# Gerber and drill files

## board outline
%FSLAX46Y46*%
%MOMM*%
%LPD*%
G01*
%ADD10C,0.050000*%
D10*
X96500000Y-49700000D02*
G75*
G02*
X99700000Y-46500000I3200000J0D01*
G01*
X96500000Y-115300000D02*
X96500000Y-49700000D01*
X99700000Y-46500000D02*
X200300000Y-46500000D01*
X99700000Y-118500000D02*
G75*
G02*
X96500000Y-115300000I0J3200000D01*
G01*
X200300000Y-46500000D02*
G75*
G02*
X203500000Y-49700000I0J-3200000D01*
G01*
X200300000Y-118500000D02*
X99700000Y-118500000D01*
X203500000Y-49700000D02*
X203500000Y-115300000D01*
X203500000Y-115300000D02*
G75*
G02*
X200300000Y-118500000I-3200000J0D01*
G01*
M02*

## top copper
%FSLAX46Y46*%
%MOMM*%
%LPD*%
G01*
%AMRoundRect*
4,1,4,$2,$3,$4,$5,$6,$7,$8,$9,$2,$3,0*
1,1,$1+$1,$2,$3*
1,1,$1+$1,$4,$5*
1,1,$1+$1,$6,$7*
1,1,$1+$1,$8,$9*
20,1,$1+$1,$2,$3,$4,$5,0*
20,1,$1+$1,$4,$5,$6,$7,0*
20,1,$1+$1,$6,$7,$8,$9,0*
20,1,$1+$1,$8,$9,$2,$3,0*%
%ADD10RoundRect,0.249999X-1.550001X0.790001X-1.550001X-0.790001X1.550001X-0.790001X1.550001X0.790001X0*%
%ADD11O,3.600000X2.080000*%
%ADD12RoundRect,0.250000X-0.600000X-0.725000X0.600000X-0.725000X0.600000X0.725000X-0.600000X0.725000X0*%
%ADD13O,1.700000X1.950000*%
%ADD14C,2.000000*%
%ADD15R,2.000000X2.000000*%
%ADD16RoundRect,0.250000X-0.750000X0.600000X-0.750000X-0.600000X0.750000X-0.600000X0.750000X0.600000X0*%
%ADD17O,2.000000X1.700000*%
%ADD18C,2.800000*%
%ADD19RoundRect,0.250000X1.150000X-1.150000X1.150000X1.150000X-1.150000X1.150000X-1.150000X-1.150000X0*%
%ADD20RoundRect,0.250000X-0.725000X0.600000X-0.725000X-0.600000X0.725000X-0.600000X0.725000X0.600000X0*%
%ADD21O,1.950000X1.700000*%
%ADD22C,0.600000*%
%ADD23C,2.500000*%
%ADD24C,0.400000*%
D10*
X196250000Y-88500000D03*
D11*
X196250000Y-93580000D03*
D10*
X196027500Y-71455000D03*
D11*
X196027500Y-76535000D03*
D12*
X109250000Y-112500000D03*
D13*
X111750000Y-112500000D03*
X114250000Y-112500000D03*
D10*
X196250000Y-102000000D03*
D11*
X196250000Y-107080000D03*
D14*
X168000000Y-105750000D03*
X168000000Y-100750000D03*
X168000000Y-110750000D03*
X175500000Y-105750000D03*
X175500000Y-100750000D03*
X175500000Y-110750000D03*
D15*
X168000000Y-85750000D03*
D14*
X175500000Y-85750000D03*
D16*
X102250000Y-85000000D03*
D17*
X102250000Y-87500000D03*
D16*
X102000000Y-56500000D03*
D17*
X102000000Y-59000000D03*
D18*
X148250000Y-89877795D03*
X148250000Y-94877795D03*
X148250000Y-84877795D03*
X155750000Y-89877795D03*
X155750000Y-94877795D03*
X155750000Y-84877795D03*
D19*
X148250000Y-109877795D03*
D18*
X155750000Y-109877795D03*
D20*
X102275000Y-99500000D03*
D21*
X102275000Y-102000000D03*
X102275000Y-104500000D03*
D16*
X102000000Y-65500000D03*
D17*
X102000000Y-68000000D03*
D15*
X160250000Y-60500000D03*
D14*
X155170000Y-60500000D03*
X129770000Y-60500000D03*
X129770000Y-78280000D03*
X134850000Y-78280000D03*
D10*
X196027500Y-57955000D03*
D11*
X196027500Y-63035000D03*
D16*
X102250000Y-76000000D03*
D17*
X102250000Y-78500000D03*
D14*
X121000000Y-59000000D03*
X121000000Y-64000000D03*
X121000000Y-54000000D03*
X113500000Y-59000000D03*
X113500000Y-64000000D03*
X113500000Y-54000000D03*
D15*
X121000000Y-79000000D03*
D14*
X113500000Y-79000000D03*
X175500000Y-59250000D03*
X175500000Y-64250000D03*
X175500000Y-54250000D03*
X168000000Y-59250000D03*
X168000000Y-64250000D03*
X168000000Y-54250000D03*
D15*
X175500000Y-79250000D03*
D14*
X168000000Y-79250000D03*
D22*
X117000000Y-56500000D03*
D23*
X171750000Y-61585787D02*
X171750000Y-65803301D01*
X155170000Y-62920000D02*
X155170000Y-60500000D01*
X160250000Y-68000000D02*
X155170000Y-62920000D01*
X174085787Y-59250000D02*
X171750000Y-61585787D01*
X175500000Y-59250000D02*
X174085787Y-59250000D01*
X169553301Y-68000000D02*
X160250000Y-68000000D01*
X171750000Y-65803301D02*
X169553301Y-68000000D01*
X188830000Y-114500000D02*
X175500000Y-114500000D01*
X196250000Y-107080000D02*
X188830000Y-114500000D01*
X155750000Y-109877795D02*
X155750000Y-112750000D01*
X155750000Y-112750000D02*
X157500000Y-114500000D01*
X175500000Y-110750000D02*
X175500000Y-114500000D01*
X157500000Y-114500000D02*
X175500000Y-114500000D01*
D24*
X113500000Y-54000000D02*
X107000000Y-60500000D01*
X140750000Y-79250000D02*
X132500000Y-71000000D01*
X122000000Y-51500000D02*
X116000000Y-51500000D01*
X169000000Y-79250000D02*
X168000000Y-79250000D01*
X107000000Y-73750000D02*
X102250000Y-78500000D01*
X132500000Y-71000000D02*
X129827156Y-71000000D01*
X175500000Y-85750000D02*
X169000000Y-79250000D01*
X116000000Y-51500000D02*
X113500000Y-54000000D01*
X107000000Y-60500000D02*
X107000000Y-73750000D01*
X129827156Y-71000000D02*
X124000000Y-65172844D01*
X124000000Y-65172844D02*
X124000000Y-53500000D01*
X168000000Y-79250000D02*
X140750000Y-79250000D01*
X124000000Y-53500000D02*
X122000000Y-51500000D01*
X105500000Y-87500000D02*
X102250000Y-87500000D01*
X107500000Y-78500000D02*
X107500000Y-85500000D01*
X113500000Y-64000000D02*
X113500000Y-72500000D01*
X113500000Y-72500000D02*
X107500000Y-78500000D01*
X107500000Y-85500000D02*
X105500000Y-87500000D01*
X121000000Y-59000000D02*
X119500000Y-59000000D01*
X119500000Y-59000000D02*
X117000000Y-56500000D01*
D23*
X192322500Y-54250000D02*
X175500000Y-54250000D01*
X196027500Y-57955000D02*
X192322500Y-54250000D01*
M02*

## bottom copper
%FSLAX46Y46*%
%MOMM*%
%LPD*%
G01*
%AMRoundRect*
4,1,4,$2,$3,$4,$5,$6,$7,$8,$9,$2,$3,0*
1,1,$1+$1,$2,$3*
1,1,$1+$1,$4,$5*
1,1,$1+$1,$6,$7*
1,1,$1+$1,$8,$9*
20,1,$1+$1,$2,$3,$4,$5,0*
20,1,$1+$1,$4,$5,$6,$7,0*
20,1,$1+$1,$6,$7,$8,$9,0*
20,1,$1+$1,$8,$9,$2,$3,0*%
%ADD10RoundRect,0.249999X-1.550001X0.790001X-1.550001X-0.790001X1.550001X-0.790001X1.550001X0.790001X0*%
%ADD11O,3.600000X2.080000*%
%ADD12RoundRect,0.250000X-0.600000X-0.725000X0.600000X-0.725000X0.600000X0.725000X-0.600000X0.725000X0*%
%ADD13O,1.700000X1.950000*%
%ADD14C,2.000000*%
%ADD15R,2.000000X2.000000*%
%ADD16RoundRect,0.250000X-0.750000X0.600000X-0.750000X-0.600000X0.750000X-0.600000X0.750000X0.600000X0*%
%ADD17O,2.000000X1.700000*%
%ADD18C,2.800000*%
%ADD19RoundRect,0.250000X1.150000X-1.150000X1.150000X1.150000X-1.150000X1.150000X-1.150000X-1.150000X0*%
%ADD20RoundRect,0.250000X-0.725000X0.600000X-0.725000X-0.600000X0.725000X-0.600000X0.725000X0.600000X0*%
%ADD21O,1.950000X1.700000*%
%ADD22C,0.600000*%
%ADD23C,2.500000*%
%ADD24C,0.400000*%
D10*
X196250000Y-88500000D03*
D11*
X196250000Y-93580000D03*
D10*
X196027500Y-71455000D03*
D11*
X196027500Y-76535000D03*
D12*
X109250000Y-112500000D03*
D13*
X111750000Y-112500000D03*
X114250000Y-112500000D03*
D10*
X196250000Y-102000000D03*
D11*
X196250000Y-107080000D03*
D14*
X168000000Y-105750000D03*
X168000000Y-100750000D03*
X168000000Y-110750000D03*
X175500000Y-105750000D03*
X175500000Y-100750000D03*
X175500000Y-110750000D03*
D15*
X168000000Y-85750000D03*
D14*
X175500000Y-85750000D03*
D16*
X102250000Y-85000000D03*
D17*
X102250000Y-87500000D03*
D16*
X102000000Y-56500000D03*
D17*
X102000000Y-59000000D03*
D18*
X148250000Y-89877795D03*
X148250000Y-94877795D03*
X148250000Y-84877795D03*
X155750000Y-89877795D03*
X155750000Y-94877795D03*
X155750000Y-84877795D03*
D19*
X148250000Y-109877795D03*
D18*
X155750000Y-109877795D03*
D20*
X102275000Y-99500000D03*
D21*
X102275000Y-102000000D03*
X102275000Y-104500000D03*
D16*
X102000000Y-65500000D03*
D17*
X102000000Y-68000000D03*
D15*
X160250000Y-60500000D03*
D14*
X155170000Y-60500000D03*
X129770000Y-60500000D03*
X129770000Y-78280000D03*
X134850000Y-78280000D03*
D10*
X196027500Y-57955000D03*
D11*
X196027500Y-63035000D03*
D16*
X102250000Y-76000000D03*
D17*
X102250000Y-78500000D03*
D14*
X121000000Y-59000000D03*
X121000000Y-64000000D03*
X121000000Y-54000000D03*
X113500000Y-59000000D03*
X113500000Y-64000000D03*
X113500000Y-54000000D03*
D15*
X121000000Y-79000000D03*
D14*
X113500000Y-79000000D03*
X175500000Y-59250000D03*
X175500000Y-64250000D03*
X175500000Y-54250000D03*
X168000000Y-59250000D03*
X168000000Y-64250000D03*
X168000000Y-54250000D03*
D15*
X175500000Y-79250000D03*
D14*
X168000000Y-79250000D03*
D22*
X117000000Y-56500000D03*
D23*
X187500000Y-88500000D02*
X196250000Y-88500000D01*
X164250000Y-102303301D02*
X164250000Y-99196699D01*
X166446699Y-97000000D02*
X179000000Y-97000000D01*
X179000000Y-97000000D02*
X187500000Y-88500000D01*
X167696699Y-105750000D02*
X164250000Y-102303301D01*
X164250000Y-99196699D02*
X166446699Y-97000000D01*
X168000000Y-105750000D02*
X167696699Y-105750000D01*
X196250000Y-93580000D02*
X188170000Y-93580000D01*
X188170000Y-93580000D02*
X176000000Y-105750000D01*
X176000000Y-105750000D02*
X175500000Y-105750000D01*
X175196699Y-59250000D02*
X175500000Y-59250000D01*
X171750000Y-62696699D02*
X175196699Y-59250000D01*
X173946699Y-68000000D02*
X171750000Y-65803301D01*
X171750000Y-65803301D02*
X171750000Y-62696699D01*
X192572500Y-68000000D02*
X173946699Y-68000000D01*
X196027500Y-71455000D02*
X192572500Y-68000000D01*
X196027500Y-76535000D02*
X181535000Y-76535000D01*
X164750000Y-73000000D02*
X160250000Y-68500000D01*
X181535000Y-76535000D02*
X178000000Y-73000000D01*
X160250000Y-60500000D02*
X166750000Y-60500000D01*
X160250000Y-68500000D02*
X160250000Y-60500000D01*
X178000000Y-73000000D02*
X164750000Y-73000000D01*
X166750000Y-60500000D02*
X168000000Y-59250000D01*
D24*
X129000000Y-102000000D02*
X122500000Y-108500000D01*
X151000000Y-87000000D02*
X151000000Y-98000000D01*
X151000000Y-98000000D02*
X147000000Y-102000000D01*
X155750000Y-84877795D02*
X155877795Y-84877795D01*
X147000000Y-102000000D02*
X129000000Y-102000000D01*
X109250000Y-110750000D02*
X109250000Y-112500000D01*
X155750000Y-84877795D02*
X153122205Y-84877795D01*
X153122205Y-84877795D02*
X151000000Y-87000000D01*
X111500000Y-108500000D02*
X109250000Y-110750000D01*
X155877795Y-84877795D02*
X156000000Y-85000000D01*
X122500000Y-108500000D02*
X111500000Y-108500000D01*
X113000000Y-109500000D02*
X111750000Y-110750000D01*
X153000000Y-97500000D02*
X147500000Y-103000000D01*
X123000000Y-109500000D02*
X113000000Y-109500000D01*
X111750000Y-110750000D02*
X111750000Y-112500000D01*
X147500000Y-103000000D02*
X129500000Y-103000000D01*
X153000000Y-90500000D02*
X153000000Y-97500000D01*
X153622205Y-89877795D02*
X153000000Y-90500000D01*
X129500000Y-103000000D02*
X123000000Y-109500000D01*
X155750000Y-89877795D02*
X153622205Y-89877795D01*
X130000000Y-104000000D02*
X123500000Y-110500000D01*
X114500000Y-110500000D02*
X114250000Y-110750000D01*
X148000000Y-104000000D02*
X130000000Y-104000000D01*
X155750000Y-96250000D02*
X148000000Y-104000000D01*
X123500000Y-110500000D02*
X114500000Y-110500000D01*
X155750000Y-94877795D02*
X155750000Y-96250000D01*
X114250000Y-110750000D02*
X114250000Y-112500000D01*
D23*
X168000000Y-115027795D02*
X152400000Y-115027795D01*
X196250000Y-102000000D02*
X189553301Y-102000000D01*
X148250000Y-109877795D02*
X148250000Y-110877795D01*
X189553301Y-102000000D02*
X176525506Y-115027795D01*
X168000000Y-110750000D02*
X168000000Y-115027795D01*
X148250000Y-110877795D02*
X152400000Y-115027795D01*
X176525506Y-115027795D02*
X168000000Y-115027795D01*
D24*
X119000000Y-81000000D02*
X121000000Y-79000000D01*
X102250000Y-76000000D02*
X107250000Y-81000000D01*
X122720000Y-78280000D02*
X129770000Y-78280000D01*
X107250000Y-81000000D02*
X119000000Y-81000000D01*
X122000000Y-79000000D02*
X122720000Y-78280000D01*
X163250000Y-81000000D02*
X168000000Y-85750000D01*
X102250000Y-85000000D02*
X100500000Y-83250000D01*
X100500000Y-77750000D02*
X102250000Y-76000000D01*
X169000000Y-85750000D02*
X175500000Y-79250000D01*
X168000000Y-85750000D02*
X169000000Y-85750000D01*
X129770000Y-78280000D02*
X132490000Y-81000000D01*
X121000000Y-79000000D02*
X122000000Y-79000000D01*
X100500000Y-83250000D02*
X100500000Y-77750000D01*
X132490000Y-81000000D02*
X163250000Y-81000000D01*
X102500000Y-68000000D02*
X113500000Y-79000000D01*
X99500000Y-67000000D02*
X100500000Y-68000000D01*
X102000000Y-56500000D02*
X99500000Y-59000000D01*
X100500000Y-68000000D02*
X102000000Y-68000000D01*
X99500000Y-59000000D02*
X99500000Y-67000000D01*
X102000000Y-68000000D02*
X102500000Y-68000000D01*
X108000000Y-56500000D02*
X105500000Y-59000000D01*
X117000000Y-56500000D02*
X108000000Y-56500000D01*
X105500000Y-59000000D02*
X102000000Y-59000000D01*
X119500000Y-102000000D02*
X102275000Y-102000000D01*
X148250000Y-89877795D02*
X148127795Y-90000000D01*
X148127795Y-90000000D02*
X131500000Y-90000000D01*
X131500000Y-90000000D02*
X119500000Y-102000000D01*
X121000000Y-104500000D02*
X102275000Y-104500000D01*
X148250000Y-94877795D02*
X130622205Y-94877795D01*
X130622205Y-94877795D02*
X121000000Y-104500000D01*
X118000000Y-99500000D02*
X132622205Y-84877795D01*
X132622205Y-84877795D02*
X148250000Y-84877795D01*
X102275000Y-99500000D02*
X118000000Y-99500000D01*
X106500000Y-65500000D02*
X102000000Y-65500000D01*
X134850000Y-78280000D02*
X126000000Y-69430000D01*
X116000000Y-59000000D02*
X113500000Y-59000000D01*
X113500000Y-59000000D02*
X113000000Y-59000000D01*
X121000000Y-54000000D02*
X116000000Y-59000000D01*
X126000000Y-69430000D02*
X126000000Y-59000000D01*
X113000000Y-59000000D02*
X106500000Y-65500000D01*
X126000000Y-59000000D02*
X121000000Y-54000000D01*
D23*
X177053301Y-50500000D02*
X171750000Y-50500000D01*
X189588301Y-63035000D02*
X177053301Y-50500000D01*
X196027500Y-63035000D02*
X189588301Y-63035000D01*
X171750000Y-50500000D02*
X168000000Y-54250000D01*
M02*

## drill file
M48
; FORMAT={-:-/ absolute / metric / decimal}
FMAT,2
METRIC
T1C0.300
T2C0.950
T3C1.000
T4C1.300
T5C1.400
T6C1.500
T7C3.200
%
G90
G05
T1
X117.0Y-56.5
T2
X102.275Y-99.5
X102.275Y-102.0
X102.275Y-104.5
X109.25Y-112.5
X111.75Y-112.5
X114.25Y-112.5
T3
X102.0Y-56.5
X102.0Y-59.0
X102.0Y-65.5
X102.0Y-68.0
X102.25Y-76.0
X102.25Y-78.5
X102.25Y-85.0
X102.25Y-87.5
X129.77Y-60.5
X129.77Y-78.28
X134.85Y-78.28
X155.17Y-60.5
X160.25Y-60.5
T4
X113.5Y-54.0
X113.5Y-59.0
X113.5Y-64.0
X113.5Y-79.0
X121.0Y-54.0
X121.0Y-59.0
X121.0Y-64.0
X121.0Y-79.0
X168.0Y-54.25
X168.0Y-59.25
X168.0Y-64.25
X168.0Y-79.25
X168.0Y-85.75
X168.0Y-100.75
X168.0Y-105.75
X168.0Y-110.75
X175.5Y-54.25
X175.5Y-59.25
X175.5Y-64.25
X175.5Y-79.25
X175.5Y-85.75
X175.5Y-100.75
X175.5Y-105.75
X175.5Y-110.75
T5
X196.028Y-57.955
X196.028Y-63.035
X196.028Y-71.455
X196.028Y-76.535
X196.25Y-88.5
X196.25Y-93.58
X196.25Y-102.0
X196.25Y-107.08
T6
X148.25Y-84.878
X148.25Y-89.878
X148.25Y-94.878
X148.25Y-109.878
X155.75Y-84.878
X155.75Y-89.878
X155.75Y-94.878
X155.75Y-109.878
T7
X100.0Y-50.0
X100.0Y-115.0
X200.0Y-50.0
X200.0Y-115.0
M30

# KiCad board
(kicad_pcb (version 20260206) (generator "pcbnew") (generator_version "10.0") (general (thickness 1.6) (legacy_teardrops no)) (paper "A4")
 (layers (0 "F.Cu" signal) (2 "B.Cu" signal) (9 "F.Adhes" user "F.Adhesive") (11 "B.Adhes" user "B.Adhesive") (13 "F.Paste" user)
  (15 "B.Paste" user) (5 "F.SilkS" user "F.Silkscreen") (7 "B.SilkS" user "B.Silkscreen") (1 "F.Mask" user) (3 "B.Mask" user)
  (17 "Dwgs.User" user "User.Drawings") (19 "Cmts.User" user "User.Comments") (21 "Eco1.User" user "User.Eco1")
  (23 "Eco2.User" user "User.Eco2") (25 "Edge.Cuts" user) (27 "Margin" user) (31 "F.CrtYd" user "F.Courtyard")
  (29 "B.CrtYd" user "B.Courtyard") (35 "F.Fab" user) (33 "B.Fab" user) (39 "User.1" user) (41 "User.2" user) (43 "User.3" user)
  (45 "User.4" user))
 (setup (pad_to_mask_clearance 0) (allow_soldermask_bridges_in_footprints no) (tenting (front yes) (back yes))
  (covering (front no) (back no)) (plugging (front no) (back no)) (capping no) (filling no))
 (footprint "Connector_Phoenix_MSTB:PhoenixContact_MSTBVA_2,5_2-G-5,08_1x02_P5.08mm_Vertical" (layer "F.Cu") (at 196.25 88.5 -90)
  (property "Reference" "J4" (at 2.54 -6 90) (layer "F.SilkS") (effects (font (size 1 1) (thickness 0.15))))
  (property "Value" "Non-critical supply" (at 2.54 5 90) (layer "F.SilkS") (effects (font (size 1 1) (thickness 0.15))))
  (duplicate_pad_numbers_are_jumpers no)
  (pad "1" thru_hole roundrect (at 0 0 270) (size 2.08 3.6) (drill 1.4) (layers "*.Cu" "*.Mask") (remove_unused_layers no)
   (roundrect_rratio 0.120192) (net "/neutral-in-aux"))
  (pad "2" thru_hole oval (at 5.08 0 270) (size 2.08 3.6) (drill 1.4) (layers "*.Cu" "*.Mask") (remove_unused_layers no)
   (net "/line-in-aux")))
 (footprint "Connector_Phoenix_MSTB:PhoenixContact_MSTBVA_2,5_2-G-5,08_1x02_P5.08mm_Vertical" (layer "F.Cu") (at 196.0275 71.455 -90)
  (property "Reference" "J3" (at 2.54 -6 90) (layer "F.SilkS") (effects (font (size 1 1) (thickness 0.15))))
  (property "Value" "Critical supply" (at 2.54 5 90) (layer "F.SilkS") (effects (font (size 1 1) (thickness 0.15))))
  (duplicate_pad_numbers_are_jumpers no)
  (pad "1" thru_hole roundrect (at 0 0 270) (size 2.08 3.6) (drill 1.4) (layers "*.Cu" "*.Mask") (remove_unused_layers no)
   (roundrect_rratio 0.120192) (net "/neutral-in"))
  (pad "2" thru_hole oval (at 5.08 0 270) (size 2.08 3.6) (drill 1.4) (layers "*.Cu" "*.Mask") (remove_unused_layers no) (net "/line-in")))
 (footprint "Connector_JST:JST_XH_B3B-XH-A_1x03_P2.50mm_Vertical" (layer "F.Cu") (at 109.25 112.5)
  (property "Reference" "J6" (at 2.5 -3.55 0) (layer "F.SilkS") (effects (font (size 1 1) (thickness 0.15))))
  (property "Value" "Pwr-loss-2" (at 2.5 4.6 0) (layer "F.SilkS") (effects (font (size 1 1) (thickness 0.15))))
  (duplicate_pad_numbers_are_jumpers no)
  (pad "1" thru_hole roundrect (at 0 0) (size 1.7 1.95) (drill 0.95) (layers "*.Cu" "*.Mask") (remove_unused_layers no)
   (roundrect_rratio 0.147059) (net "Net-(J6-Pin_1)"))
  (pad "2" thru_hole oval (at 2.5 0) (size 1.7 1.95) (drill 0.95) (layers "*.Cu" "*.Mask") (remove_unused_layers no) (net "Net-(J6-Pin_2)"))
  (pad "3" thru_hole oval (at 5 0) (size 1.7 1.95) (drill 0.95) (layers "*.Cu" "*.Mask") (remove_unused_layers no) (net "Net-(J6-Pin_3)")))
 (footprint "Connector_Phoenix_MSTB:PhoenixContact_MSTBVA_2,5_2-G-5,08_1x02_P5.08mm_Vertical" (layer "F.Cu") (at 196.25 102 -90)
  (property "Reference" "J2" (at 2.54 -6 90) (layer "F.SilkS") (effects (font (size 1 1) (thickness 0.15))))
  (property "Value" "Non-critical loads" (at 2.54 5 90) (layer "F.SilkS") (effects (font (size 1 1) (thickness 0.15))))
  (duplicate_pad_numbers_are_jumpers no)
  (pad "1" thru_hole roundrect (at 0 0 270) (size 2.08 3.6) (drill 1.4) (layers "*.Cu" "*.Mask") (remove_unused_layers no)
   (roundrect_rratio 0.120192) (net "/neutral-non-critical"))
  (pad "2" thru_hole oval (at 5.08 0 270) (size 2.08 3.6) (drill 1.4) (layers "*.Cu" "*.Mask") (remove_unused_layers no)
   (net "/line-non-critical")))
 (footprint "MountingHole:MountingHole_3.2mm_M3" (layer "F.Cu") (at 200 50)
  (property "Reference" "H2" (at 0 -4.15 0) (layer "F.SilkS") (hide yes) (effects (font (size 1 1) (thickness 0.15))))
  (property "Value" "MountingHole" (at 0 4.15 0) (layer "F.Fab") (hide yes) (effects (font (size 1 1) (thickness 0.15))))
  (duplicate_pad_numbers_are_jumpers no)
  (pad "" np_thru_hole circle (at 0 0) (size 3.2 3.2) (drill 3.2) (layers "*.Cu" "*.Mask")))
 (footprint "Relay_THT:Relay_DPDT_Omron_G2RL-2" (layer "F.Cu") (at 168 85.75)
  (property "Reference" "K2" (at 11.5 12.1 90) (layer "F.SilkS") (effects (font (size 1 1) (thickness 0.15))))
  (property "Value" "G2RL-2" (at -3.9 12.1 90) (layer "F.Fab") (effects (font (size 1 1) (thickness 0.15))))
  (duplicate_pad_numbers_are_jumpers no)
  (pad "11" thru_hole circle (at 0 20) (size 2 2) (drill 1.3) (layers "*.Cu" "*.Mask") (remove_unused_layers no) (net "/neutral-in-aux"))
  (pad "12" thru_hole circle (at 0 15) (size 2 2) (drill 1.3) (layers "*.Cu" "*.Mask") (remove_unused_layers no)
   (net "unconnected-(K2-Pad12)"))
  (pad "14" thru_hole circle (at 0 25) (size 2 2) (drill 1.3) (layers "*.Cu" "*.Mask") (remove_unused_layers no)
   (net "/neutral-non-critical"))
  (pad "21" thru_hole circle (at 7.5 20) (size 2 2) (drill 1.3) (layers "*.Cu" "*.Mask") (remove_unused_layers no) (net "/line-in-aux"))
  (pad "22" thru_hole circle (at 7.5 15) (size 2 2) (drill 1.3) (layers "*.Cu" "*.Mask") (remove_unused_layers no)
   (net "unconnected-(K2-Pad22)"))
  (pad "24" thru_hole circle (at 7.5 25) (size 2 2) (drill 1.3) (layers "*.Cu" "*.Mask") (remove_unused_layers no)
   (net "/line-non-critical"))
  (pad "A1" thru_hole rect (at 0 0) (size 2 2) (drill 1.3) (layers "*.Cu" "*.Mask") (remove_unused_layers no) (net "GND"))
  (pad "A2" thru_hole circle (at 7.5 0) (size 2 2) (drill 1.3) (layers "*.Cu" "*.Mask") (remove_unused_layers no) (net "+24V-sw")))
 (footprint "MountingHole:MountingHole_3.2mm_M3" (layer "F.Cu") (at 100 50)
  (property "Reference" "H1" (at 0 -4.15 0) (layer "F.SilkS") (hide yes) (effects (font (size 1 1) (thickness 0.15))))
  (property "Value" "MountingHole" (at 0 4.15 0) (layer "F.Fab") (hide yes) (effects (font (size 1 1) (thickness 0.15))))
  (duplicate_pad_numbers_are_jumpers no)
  (pad "" np_thru_hole circle (at 0 0) (size 3.2 3.2) (drill 3.2) (layers "*.Cu" "*.Mask")))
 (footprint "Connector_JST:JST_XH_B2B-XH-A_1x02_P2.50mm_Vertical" (layer "F.Cu") (at 102.25 85 -90)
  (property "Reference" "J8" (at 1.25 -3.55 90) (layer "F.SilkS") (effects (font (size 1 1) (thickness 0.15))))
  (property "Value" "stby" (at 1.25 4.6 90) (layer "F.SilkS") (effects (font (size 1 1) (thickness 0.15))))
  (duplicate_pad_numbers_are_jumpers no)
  (pad "1" thru_hole roundrect (at 0 0 270) (size 1.7 2) (drill 1) (layers "*.Cu" "*.Mask") (remove_unused_layers no)
   (roundrect_rratio 0.147059) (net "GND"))
  (pad "2" thru_hole oval (at 2.5 0 270) (size 1.7 2) (drill 1) (layers "*.Cu" "*.Mask") (remove_unused_layers no) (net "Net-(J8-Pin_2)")))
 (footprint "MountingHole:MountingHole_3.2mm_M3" (layer "F.Cu") (at 200 115)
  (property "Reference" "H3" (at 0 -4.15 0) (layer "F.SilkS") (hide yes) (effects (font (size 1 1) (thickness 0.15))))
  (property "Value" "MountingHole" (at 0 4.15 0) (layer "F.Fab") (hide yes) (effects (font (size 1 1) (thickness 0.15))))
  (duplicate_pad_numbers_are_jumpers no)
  (pad "" np_thru_hole circle (at 0 0) (size 3.2 3.2) (drill 3.2) (layers "*.Cu" "*.Mask")))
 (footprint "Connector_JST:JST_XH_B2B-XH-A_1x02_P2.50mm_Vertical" (layer "F.Cu") (at 102 56.5 -90)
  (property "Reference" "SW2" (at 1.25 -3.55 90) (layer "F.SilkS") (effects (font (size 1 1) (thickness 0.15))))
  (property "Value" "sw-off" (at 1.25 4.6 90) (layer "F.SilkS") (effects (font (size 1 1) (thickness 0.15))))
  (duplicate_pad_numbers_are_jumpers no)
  (pad "1" thru_hole roundrect (at 0 0 270) (size 1.7 2) (drill 1) (layers "*.Cu" "*.Mask") (remove_unused_layers no)
   (roundrect_rratio 0.147059) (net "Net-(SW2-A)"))
  (pad "2" thru_hole oval (at 2.5 0 270) (size 1.7 2) (drill 1) (layers "*.Cu" "*.Mask") (remove_unused_layers no) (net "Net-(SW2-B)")))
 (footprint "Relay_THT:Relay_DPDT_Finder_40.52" (layer "F.Cu") (at 148.25 109.877795 90)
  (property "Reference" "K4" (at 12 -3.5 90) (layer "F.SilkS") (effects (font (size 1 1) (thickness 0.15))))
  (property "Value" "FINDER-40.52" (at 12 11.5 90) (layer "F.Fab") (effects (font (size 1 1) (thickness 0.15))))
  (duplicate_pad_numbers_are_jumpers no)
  (pad "11" thru_hole circle (at 20 0 90) (size 2.8 2.8) (drill 1.5) (layers "*.Cu" "*.Mask") (remove_unused_layers no)
   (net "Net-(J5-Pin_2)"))
  (pad "12" thru_hole circle (at 15 0 90) (size 2.8 2.8) (drill 1.5) (layers "*.Cu" "*.Mask") (remove_unused_layers no)
   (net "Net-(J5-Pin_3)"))
  (pad "14" thru_hole circle (at 25 0 90) (size 2.8 2.8) (drill 1.5) (layers "*.Cu" "*.Mask") (remove_unused_layers no)
   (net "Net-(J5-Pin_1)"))
  (pad "21" thru_hole circle (at 20 7.5 90) (size 2.8 2.8) (drill 1.5) (layers "*.Cu" "*.Mask") (remove_unused_layers no)
   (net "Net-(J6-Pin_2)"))
  (pad "22" thru_hole circle (at 15 7.5 90) (size 2.8 2.8) (drill 1.5) (layers "*.Cu" "*.Mask") (remove_unused_layers no)
   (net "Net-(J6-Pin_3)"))
  (pad "24" thru_hole circle (at 25 7.5 90) (size 2.8 2.8) (drill 1.5) (layers "*.Cu" "*.Mask") (remove_unused_layers no)
   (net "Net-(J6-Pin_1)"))
  (pad "A1" thru_hole roundrect (at 0 0 90) (size 2.8 2.8) (drill 1.5) (layers "*.Cu" "*.Mask") (remove_unused_layers no)
   (roundrect_rratio 0.08928571429) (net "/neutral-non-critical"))
  (pad "A2" thru_hole circle (at 0 7.5 90) (size 2.8 2.8) (drill 1.5) (layers "*.Cu" "*.Mask") (remove_unused_layers no)
   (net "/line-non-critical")))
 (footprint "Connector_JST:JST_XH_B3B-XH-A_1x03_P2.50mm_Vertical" (layer "F.Cu") (at 102.275 99.5 -90)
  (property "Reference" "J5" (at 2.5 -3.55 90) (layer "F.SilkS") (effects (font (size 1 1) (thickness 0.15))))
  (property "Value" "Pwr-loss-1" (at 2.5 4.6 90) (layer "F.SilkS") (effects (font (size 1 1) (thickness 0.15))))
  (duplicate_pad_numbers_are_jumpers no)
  (pad "1" thru_hole roundrect (at 0 0 270) (size 1.7 1.95) (drill 0.95) (layers "*.Cu" "*.Mask") (remove_unused_layers no)
   (roundrect_rratio 0.147059) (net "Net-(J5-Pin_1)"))
  (pad "2" thru_hole oval (at 2.5 0 270) (size 1.7 1.95) (drill 0.95) (layers "*.Cu" "*.Mask") (remove_unused_layers no)
   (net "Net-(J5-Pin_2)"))
  (pad "3" thru_hole oval (at 5 0 270) (size 1.7 1.95) (drill 0.95) (layers "*.Cu" "*.Mask") (remove_unused_layers no)
   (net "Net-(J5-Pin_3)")))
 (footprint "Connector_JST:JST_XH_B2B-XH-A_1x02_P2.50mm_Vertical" (layer "F.Cu") (at 102 65.5 -90)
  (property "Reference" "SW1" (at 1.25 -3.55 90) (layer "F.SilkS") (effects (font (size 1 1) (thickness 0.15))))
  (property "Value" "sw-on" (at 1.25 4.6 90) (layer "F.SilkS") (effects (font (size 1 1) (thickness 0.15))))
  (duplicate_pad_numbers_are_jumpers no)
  (pad "1" thru_hole roundrect (at 0 0 270) (size 1.7 2) (drill 1) (layers "*.Cu" "*.Mask") (remove_unused_layers no)
   (roundrect_rratio 0.147059) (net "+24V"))
  (pad "2" thru_hole oval (at 2.5 0 270) (size 1.7 2) (drill 1) (layers "*.Cu" "*.Mask") (remove_unused_layers no) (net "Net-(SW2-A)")))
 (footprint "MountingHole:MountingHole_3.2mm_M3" (layer "F.Cu") (at 100 115)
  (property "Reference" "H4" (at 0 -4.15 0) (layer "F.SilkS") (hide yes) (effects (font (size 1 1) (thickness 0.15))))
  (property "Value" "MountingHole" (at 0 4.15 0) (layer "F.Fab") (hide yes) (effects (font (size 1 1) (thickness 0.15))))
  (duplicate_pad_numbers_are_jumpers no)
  (pad "" np_thru_hole circle (at 0 0) (size 3.2 3.2) (drill 3.2) (layers "*.Cu" "*.Mask")))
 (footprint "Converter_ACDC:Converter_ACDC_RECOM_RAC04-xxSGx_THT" (layer "F.Cu") (at 160.25 60.5 -90)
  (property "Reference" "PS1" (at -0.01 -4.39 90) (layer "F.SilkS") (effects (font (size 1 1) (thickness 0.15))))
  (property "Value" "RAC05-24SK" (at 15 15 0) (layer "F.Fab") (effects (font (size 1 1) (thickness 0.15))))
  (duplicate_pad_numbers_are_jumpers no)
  (pad "1" thru_hole rect (at 0 0) (size 2 2) (drill 1) (layers "*.Cu" "*.Mask") (remove_unused_layers no) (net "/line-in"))
  (pad "2" thru_hole circle (at 0 5.08) (size 2 2) (drill 1) (layers "*.Cu" "*.Mask") (remove_unused_layers no) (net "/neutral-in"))
  (pad "3" thru_hole circle (at 0 30.48 90) (size 2 2) (drill 1) (layers "*.Cu" "*.Mask") (remove_unused_layers no)
   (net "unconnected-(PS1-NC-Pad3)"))
  (pad "4" thru_hole circle (at 17.78 30.48) (size 2 2) (drill 1) (layers "*.Cu" "*.Mask") (remove_unused_layers no) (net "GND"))
  (pad "5" thru_hole circle (at 17.78 25.4) (size 2 2) (drill 1) (layers "*.Cu" "*.Mask") (remove_unused_layers no) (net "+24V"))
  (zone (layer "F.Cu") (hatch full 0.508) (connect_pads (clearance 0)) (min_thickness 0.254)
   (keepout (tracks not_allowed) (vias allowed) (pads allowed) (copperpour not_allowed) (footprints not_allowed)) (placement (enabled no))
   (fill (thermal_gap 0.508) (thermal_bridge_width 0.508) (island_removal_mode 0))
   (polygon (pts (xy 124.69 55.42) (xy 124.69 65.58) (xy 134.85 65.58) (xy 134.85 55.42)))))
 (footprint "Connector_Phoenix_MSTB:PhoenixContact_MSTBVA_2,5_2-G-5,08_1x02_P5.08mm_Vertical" (layer "F.Cu") (at 196.0275 57.955 -90)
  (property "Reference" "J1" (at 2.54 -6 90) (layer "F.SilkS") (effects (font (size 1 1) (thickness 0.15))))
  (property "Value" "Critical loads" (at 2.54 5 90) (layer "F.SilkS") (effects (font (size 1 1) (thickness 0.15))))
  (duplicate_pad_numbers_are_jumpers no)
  (pad "1" thru_hole roundrect (at 0 0 270) (size 2.08 3.6) (drill 1.4) (layers "*.Cu" "*.Mask") (remove_unused_layers no)
   (roundrect_rratio 0.120192) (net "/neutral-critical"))
  (pad "2" thru_hole oval (at 5.08 0 270) (size 2.08 3.6) (drill 1.4) (layers "*.Cu" "*.Mask") (remove_unused_layers no)
   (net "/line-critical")))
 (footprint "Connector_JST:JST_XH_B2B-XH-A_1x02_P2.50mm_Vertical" (layer "F.Cu") (at 102.25 76 -90)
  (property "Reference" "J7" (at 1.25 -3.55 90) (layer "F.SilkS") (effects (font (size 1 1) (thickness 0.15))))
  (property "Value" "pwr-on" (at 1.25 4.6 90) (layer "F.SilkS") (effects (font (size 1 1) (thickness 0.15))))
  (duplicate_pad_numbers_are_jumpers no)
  (pad "1" thru_hole roundrect (at 0 0 270) (size 1.7 2) (drill 1) (layers "*.Cu" "*.Mask") (remove_unused_layers no)
   (roundrect_rratio 0.147059) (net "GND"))
  (pad "2" thru_hole oval (at 2.5 0 270) (size 1.7 2) (drill 1) (layers "*.Cu" "*.Mask") (remove_unused_layers no) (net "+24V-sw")))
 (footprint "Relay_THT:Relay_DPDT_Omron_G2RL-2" (layer "F.Cu") (at 121 79 180)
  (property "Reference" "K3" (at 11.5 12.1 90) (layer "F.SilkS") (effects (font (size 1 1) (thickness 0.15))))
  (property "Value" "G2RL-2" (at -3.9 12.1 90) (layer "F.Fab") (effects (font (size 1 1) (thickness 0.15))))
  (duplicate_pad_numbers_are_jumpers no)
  (pad "11" thru_hole circle (at 0 20 180) (size 2 2) (drill 1.3) (layers "*.Cu" "*.Mask") (remove_unused_layers no) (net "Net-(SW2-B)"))
  (pad "12" thru_hole circle (at 0 15 180) (size 2 2) (drill 1.3) (layers "*.Cu" "*.Mask") (remove_unused_layers no)
   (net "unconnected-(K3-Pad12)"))
  (pad "14" thru_hole circle (at 0 25 180) (size 2 2) (drill 1.3) (layers "*.Cu" "*.Mask") (remove_unused_layers no) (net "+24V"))
  (pad "21" thru_hole circle (at 7.5 20 180) (size 2 2) (drill 1.3) (layers "*.Cu" "*.Mask") (remove_unused_layers no) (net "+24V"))
  (pad "22" thru_hole circle (at 7.5 15 180) (size 2 2) (drill 1.3) (layers "*.Cu" "*.Mask") (remove_unused_layers no)
   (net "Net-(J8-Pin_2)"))
  (pad "24" thru_hole circle (at 7.5 25 180) (size 2 2) (drill 1.3) (layers "*.Cu" "*.Mask") (remove_unused_layers no) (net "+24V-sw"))
  (pad "A1" thru_hole rect (at 0 0 180) (size 2 2) (drill 1.3) (layers "*.Cu" "*.Mask") (remove_unused_layers no) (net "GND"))
  (pad "A2" thru_hole circle (at 7.5 0 180) (size 2 2) (drill 1.3) (layers "*.Cu" "*.Mask") (remove_unused_layers no) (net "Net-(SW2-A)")))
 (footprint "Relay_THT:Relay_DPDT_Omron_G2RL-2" (layer "F.Cu") (at 175.5 79.25 180)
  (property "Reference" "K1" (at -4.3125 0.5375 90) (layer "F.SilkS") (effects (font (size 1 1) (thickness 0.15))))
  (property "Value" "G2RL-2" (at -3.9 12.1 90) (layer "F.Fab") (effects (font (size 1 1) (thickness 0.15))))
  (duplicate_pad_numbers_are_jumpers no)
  (pad "11" thru_hole circle (at 0 20 180) (size 2 2) (drill 1.3) (layers "*.Cu" "*.Mask") (remove_unused_layers no) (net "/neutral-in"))
  (pad "12" thru_hole circle (at 0 15 180) (size 2 2) (drill 1.3) (layers "*.Cu" "*.Mask") (remove_unused_layers no)
   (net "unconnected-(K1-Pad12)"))
  (pad "14" thru_hole circle (at 0 25 180) (size 2 2) (drill 1.3) (layers "*.Cu" "*.Mask") (remove_unused_layers no)
   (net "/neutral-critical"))
  (pad "21" thru_hole circle (at 7.5 20 180) (size 2 2) (drill 1.3) (layers "*.Cu" "*.Mask") (remove_unused_layers no) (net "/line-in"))
  (pad "22" thru_hole circle (at 7.5 15 180) (size 2 2) (drill 1.3) (layers "*.Cu" "*.Mask") (remove_unused_layers no)
   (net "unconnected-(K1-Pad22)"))
  (pad "24" thru_hole circle (at 7.5 25 180) (size 2 2) (drill 1.3) (layers "*.Cu" "*.Mask") (remove_unused_layers no)
   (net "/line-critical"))
  (pad "A1" thru_hole rect (at 0 0 180) (size 2 2) (drill 1.3) (layers "*.Cu" "*.Mask") (remove_unused_layers no) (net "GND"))
  (pad "A2" thru_hole circle (at 7.5 0 180) (size 2 2) (drill 1.3) (layers "*.Cu" "*.Mask") (remove_unused_layers no) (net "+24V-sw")))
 (gr_arc (start 96.5 49.7) (mid 97.437258 47.437258) (end 99.7 46.5) (stroke (width 0.05) (type default)) (layer "Edge.Cuts"))
 (gr_line (start 96.5 115.3) (end 96.5 49.7) (stroke (width 0.05) (type default)) (layer "Edge.Cuts"))
 (gr_line (start 99.7 46.5) (end 200.3 46.5) (stroke (width 0.05) (type default)) (layer "Edge.Cuts"))
 (gr_arc (start 99.7 118.5) (mid 97.437258 117.562742) (end 96.5 115.3) (stroke (width 0.05) (type default)) (layer "Edge.Cuts"))
 (gr_arc (start 200.3 46.5) (mid 202.562742 47.437258) (end 203.5 49.7) (stroke (width 0.05) (type default)) (layer "Edge.Cuts"))
 (gr_line (start 200.3 118.5) (end 99.7 118.5) (stroke (width 0.05) (type default)) (layer "Edge.Cuts"))
 (gr_line (start 203.5 49.7) (end 203.5 115.3) (stroke (width 0.05) (type default)) (layer "Edge.Cuts"))
 (gr_arc (start 203.5 115.3) (mid 202.562742 117.562742) (end 200.3 118.5) (stroke (width 0.05) (type default)) (layer "Edge.Cuts"))
 (segment (start 187.5 88.5) (end 196.25 88.5) (width 2.5) (layer "B.Cu") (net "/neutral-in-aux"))
 (segment (start 164.25 102.303301) (end 164.25 99.196699) (width 2.5) (layer "B.Cu") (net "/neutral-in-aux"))
 (segment (start 166.446699 97) (end 179 97) (width 2.5) (layer "B.Cu") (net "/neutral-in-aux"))
 (segment (start 179 97) (end 187.5 88.5) (width 2.5) (layer "B.Cu") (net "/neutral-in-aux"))
 (segment (start 167.696699 105.75) (end 164.25 102.303301) (width 2.5) (layer "B.Cu") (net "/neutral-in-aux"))
 (segment (start 164.25 99.196699) (end 166.446699 97) (width 2.5) (layer "B.Cu") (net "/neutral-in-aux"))
 (segment (start 168 105.75) (end 167.696699 105.75) (width 2.5) (layer "B.Cu") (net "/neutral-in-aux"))
 (segment (start 196.25 93.58) (end 188.17 93.58) (width 2.5) (layer "B.Cu") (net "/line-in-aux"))
 (segment (start 188.17 93.58) (end 176 105.75) (width 2.5) (layer "B.Cu") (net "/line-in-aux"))
 (segment (start 176 105.75) (end 175.5 105.75) (width 2.5) (layer "B.Cu") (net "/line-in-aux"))
 (segment (start 171.75 61.585787) (end 171.75 65.803301) (width 2.5) (layer "F.Cu") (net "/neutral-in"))
 (segment (start 155.17 62.92) (end 155.17 60.5) (width 2.5) (layer "F.Cu") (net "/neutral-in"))
 (segment (start 160.25 68) (end 155.17 62.92) (width 2.5) (layer "F.Cu") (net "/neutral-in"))
 (segment (start 174.085787 59.25) (end 171.75 61.585787) (width 2.5) (layer "F.Cu") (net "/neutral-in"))
 (segment (start 175.5 59.25) (end 174.085787 59.25) (width 2.5) (layer "F.Cu") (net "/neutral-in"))
 (segment (start 169.553301 68) (end 160.25 68) (width 2.5) (layer "F.Cu") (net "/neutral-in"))
 (segment (start 171.75 65.803301) (end 169.553301 68) (width 2.5) (layer "F.Cu") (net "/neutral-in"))
 (segment (start 175.196699 59.25) (end 175.5 59.25) (width 2.5) (layer "B.Cu") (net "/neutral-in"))
 (segment (start 171.75 62.696699) (end 175.196699 59.25) (width 2.5) (layer "B.Cu") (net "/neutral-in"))
 (segment (start 173.946699 68) (end 171.75 65.803301) (width 2.5) (layer "B.Cu") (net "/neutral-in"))
 (segment (start 171.75 65.803301) (end 171.75 62.696699) (width 2.5) (layer "B.Cu") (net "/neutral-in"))
 (segment (start 192.5725 68) (end 173.946699 68) (width 2.5) (layer "B.Cu") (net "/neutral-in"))
 (segment (start 196.0275 71.455) (end 192.5725 68) (width 2.5) (layer "B.Cu") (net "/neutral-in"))
 (segment (start 196.0275 76.535) (end 181.535 76.535) (width 2.5) (layer "B.Cu") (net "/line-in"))
 (segment (start 164.75 73) (end 160.25 68.5) (width 2.5) (layer "B.Cu") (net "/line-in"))
 (segment (start 181.535 76.535) (end 178 73) (width 2.5) (layer "B.Cu") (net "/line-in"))
 (segment (start 160.25 60.5) (end 166.75 60.5) (width 2.5) (layer "B.Cu") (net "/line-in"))
 (segment (start 160.25 68.5) (end 160.25 60.5) (width 2.5) (layer "B.Cu") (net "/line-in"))
 (segment (start 178 73) (end 164.75 73) (width 2.5) (layer "B.Cu") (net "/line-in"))
 (segment (start 166.75 60.5) (end 168 59.25) (width 2.5) (layer "B.Cu") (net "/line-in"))
 (segment (start 129 102) (end 122.5 108.5) (width 0.4) (layer "B.Cu") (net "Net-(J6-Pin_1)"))
 (segment (start 151 87) (end 151 98) (width 0.4) (layer "B.Cu") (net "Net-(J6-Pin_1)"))
 (segment (start 151 98) (end 147 102) (width 0.4) (layer "B.Cu") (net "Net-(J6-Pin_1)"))
 (segment (start 155.75 84.877795) (end 155.877795 84.877795) (width 0.4) (layer "B.Cu") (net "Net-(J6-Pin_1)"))
 (segment (start 147 102) (end 129 102) (width 0.4) (layer "B.Cu") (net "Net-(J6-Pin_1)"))
 (segment (start 109.25 110.75) (end 109.25 112.5) (width 0.4) (layer "B.Cu") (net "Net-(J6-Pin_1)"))
 (segment (start 155.75 84.877795) (end 153.122205 84.877795) (width 0.4) (layer "B.Cu") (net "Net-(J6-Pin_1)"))
 (segment (start 153.122205 84.877795) (end 151 87) (width 0.4) (layer "B.Cu") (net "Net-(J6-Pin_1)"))
 (segment (start 111.5 108.5) (end 109.25 110.75) (width 0.4) (layer "B.Cu") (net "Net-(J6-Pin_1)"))
 (segment (start 155.877795 84.877795) (end 156 85) (width 0.4) (layer "B.Cu") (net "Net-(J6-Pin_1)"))
 (segment (start 122.5 108.5) (end 111.5 108.5) (width 0.4) (layer "B.Cu") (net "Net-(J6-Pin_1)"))
 (segment (start 113 109.5) (end 111.75 110.75) (width 0.4) (layer "B.Cu") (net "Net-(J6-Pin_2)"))
 (segment (start 153 97.5) (end 147.5 103) (width 0.4) (layer "B.Cu") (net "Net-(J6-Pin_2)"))
 (segment (start 123 109.5) (end 113 109.5) (width 0.4) (layer "B.Cu") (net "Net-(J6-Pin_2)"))
 (segment (start 111.75 110.75) (end 111.75 112.5) (width 0.4) (layer "B.Cu") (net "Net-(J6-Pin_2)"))
 (segment (start 147.5 103) (end 129.5 103) (width 0.4) (layer "B.Cu") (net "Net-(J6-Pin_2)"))
 (segment (start 153 90.5) (end 153 97.5) (width 0.4) (layer "B.Cu") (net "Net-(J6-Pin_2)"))
 (segment (start 153.622205 89.877795) (end 153 90.5) (width 0.4) (layer "B.Cu") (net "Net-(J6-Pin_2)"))
 (segment (start 129.5 103) (end 123 109.5) (width 0.4) (layer "B.Cu") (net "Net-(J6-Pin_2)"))
 (segment (start 155.75 89.877795) (end 153.622205 89.877795) (width 0.4) (layer "B.Cu") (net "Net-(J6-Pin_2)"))
 (segment (start 130 104) (end 123.5 110.5) (width 0.4) (layer "B.Cu") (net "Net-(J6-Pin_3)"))
 (segment (start 114.5 110.5) (end 114.25 110.75) (width 0.4) (layer "B.Cu") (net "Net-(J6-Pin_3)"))
 (segment (start 148 104) (end 130 104) (width 0.4) (layer "B.Cu") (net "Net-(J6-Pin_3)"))
 (segment (start 155.75 96.25) (end 148 104) (width 0.4) (layer "B.Cu") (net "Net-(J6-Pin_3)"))
 (segment (start 123.5 110.5) (end 114.5 110.5) (width 0.4) (layer "B.Cu") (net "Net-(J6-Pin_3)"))
 (segment (start 155.75 94.877795) (end 155.75 96.25) (width 0.4) (layer "B.Cu") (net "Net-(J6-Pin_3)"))
 (segment (start 114.25 110.75) (end 114.25 112.5) (width 0.4) (layer "B.Cu") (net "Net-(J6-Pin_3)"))
 (segment (start 168 115.027795) (end 152.4 115.027795) (width 2.5) (layer "B.Cu") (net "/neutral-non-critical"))
 (segment (start 196.25 102) (end 189.553301 102) (width 2.5) (layer "B.Cu") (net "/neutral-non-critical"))
 (segment (start 148.25 109.877795) (end 148.25 110.877795) (width 2.5) (layer "B.Cu") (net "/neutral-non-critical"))
 (segment (start 189.553301 102) (end 176.525506 115.027795) (width 2.5) (layer "B.Cu") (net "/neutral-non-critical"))
 (segment (start 168 110.75) (end 168 115.027795) (width 2.5) (layer "B.Cu") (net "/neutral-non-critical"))
 (segment (start 148.25 110.877795) (end 152.4 115.027795) (width 2.5) (layer "B.Cu") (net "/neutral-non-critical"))
 (segment (start 176.525506 115.027795) (end 168 115.027795) (width 2.5) (layer "B.Cu") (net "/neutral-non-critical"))
 (segment (start 188.83 114.5) (end 175.5 114.5) (width 2.5) (layer "F.Cu") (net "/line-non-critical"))
 (segment (start 196.25 107.08) (end 188.83 114.5) (width 2.5) (layer "F.Cu") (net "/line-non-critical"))
 (segment (start 155.75 109.877795) (end 155.75 112.75) (width 2.5) (layer "F.Cu") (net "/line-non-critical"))
 (segment (start 155.75 112.75) (end 157.5 114.5) (width 2.5) (layer "F.Cu") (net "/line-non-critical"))
 (segment (start 175.5 110.75) (end 175.5 114.5) (width 2.5) (layer "F.Cu") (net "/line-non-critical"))
 (segment (start 157.5 114.5) (end 175.5 114.5) (width 2.5) (layer "F.Cu") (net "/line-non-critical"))
 (segment (start 119 81) (end 121 79) (width 0.4) (layer "B.Cu") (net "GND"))
 (segment (start 102.25 76) (end 107.25 81) (width 0.4) (layer "B.Cu") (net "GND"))
 (segment (start 122.72 78.28) (end 129.77 78.28) (width 0.4) (layer "B.Cu") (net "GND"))
 (segment (start 107.25 81) (end 119 81) (width 0.4) (layer "B.Cu") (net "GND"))
 (segment (start 122 79) (end 122.72 78.28) (width 0.4) (layer "B.Cu") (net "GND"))
 (segment (start 163.25 81) (end 168 85.75) (width 0.4) (layer "B.Cu") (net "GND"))
 (segment (start 102.25 85) (end 100.5 83.25) (width 0.4) (layer "B.Cu") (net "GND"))
 (segment (start 100.5 77.75) (end 102.25 76) (width 0.4) (layer "B.Cu") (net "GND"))
 (segment (start 169 85.75) (end 175.5 79.25) (width 0.4) (layer "B.Cu") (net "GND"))
 (segment (start 168 85.75) (end 169 85.75) (width 0.4) (layer "B.Cu") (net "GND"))
 (segment (start 129.77 78.28) (end 132.49 81) (width 0.4) (layer "B.Cu") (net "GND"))
 (segment (start 121 79) (end 122 79) (width 0.4) (layer "B.Cu") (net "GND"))
 (segment (start 100.5 83.25) (end 100.5 77.75) (width 0.4) (layer "B.Cu") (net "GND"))
 (segment (start 132.49 81) (end 163.25 81) (width 0.4) (layer "B.Cu") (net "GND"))
 (segment (start 113.5 54) (end 107 60.5) (width 0.4) (layer "F.Cu") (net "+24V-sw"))
 (segment (start 140.75 79.25) (end 132.5 71) (width 0.4) (layer "F.Cu") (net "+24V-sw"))
 (segment (start 122 51.5) (end 116 51.5) (width 0.4) (layer "F.Cu") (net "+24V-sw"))
 (segment (start 169 79.25) (end 168 79.25) (width 0.4) (layer "F.Cu") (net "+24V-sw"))
 (segment (start 107 73.75) (end 102.25 78.5) (width 0.4) (layer "F.Cu") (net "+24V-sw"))
 (segment (start 132.5 71) (end 129.827156 71) (width 0.4) (layer "F.Cu") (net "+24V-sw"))
 (segment (start 175.5 85.75) (end 169 79.25) (width 0.4) (layer "F.Cu") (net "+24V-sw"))
 (segment (start 116 51.5) (end 113.5 54) (width 0.4) (layer "F.Cu") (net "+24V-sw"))
 (segment (start 107 60.5) (end 107 73.75) (width 0.4) (layer "F.Cu") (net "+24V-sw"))
 (segment (start 129.827156 71) (end 124 65.172844) (width 0.4) (layer "F.Cu") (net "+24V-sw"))
 (segment (start 124 65.172844) (end 124 53.5) (width 0.4) (layer "F.Cu") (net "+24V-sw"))
 (segment (start 168 79.25) (end 140.75 79.25) (width 0.4) (layer "F.Cu") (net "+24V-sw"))
 (segment (start 124 53.5) (end 122 51.5) (width 0.4) (layer "F.Cu") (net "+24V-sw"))
 (segment (start 105.5 87.5) (end 102.25 87.5) (width 0.4) (layer "F.Cu") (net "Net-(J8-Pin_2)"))
 (segment (start 107.5 78.5) (end 107.5 85.5) (width 0.4) (layer "F.Cu") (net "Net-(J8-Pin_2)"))
 (segment (start 113.5 64) (end 113.5 72.5) (width 0.4) (layer "F.Cu") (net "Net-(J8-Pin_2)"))
 (segment (start 113.5 72.5) (end 107.5 78.5) (width 0.4) (layer "F.Cu") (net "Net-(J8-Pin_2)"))
 (segment (start 107.5 85.5) (end 105.5 87.5) (width 0.4) (layer "F.Cu") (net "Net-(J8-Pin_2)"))
 (segment (start 102.5 68) (end 113.5 79) (width 0.4) (layer "B.Cu") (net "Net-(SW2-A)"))
 (segment (start 99.5 67) (end 100.5 68) (width 0.4) (layer "B.Cu") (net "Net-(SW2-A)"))
 (segment (start 102 56.5) (end 99.5 59) (width 0.4) (layer "B.Cu") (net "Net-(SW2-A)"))
 (segment (start 100.5 68) (end 102 68) (width 0.4) (layer "B.Cu") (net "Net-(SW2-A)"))
 (segment (start 99.5 59) (end 99.5 67) (width 0.4) (layer "B.Cu") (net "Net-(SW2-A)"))
 (segment (start 102 68) (end 102.5 68) (width 0.4) (layer "B.Cu") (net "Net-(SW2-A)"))
 (segment (start 121 59) (end 119.5 59) (width 0.4) (layer "F.Cu") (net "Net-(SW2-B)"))
 (segment (start 119.5 59) (end 117 56.5) (width 0.4) (layer "F.Cu") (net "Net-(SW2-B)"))
 (via (at 117 56.5) (size 0.6) (drill 0.3) (layers "F.Cu" "B.Cu") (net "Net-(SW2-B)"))
 (segment (start 108 56.5) (end 105.5 59) (width 0.4) (layer "B.Cu") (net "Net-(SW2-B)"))
 (segment (start 117 56.5) (end 108 56.5) (width 0.4) (layer "B.Cu") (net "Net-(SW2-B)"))
 (segment (start 105.5 59) (end 102 59) (width 0.4) (layer "B.Cu") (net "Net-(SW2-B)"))
 (segment (start 119.5 102) (end 102.275 102) (width 0.4) (layer "B.Cu") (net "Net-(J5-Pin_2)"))
 (segment (start 148.25 89.877795) (end 148.127795 90) (width 0.4) (layer "B.Cu") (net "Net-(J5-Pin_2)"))
 (segment (start 148.127795 90) (end 131.5 90) (width 0.4) (layer "B.Cu") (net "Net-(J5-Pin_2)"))
 (segment (start 131.5 90) (end 119.5 102) (width 0.4) (layer "B.Cu") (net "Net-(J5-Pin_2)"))
 (segment (start 121 104.5) (end 102.275 104.5) (width 0.4) (layer "B.Cu") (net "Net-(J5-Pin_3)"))
 (segment (start 148.25 94.877795) (end 130.622205 94.877795) (width 0.4) (layer "B.Cu") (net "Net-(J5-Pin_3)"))
 (segment (start 130.622205 94.877795) (end 121 104.5) (width 0.4) (layer "B.Cu") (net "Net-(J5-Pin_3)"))
 (segment (start 118 99.5) (end 132.622205 84.877795) (width 0.4) (layer "B.Cu") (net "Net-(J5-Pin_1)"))
 (segment (start 132.622205 84.877795) (end 148.25 84.877795) (width 0.4) (layer "B.Cu") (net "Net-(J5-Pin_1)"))
 (segment (start 102.275 99.5) (end 118 99.5) (width 0.4) (layer "B.Cu") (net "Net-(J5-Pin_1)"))
 (segment (start 106.5 65.5) (end 102 65.5) (width 0.4) (layer "B.Cu") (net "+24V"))
 (segment (start 134.85 78.28) (end 126 69.43) (width 0.4) (layer "B.Cu") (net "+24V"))
 (segment (start 116 59) (end 113.5 59) (width 0.4) (layer "B.Cu") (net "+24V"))
 (segment (start 113.5 59) (end 113 59) (width 0.4) (layer "B.Cu") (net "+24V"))
 (segment (start 121 54) (end 116 59) (width 0.4) (layer "B.Cu") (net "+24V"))
 (segment (start 126 69.43) (end 126 59) (width 0.4) (layer "B.Cu") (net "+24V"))
 (segment (start 113 59) (end 106.5 65.5) (width 0.4) (layer "B.Cu") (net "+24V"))
 (segment (start 126 59) (end 121 54) (width 0.4) (layer "B.Cu") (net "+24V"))
 (segment (start 192.3225 54.25) (end 175.5 54.25) (width 2.5) (layer "F.Cu") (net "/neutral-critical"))
 (segment (start 196.0275 57.955) (end 192.3225 54.25) (width 2.5) (layer "F.Cu") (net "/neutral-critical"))
 (segment (start 177.053301 50.5) (end 171.75 50.5) (width 2.5) (layer "B.Cu") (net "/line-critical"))
 (segment (start 189.588301 63.035) (end 177.053301 50.5) (width 2.5) (layer "B.Cu") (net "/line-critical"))
 (segment (start 196.0275 63.035) (end 189.588301 63.035) (width 2.5) (layer "B.Cu") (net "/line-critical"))
 (segment (start 171.75 50.5) (end 168 54.25) (width 2.5) (layer "B.Cu") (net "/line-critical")))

